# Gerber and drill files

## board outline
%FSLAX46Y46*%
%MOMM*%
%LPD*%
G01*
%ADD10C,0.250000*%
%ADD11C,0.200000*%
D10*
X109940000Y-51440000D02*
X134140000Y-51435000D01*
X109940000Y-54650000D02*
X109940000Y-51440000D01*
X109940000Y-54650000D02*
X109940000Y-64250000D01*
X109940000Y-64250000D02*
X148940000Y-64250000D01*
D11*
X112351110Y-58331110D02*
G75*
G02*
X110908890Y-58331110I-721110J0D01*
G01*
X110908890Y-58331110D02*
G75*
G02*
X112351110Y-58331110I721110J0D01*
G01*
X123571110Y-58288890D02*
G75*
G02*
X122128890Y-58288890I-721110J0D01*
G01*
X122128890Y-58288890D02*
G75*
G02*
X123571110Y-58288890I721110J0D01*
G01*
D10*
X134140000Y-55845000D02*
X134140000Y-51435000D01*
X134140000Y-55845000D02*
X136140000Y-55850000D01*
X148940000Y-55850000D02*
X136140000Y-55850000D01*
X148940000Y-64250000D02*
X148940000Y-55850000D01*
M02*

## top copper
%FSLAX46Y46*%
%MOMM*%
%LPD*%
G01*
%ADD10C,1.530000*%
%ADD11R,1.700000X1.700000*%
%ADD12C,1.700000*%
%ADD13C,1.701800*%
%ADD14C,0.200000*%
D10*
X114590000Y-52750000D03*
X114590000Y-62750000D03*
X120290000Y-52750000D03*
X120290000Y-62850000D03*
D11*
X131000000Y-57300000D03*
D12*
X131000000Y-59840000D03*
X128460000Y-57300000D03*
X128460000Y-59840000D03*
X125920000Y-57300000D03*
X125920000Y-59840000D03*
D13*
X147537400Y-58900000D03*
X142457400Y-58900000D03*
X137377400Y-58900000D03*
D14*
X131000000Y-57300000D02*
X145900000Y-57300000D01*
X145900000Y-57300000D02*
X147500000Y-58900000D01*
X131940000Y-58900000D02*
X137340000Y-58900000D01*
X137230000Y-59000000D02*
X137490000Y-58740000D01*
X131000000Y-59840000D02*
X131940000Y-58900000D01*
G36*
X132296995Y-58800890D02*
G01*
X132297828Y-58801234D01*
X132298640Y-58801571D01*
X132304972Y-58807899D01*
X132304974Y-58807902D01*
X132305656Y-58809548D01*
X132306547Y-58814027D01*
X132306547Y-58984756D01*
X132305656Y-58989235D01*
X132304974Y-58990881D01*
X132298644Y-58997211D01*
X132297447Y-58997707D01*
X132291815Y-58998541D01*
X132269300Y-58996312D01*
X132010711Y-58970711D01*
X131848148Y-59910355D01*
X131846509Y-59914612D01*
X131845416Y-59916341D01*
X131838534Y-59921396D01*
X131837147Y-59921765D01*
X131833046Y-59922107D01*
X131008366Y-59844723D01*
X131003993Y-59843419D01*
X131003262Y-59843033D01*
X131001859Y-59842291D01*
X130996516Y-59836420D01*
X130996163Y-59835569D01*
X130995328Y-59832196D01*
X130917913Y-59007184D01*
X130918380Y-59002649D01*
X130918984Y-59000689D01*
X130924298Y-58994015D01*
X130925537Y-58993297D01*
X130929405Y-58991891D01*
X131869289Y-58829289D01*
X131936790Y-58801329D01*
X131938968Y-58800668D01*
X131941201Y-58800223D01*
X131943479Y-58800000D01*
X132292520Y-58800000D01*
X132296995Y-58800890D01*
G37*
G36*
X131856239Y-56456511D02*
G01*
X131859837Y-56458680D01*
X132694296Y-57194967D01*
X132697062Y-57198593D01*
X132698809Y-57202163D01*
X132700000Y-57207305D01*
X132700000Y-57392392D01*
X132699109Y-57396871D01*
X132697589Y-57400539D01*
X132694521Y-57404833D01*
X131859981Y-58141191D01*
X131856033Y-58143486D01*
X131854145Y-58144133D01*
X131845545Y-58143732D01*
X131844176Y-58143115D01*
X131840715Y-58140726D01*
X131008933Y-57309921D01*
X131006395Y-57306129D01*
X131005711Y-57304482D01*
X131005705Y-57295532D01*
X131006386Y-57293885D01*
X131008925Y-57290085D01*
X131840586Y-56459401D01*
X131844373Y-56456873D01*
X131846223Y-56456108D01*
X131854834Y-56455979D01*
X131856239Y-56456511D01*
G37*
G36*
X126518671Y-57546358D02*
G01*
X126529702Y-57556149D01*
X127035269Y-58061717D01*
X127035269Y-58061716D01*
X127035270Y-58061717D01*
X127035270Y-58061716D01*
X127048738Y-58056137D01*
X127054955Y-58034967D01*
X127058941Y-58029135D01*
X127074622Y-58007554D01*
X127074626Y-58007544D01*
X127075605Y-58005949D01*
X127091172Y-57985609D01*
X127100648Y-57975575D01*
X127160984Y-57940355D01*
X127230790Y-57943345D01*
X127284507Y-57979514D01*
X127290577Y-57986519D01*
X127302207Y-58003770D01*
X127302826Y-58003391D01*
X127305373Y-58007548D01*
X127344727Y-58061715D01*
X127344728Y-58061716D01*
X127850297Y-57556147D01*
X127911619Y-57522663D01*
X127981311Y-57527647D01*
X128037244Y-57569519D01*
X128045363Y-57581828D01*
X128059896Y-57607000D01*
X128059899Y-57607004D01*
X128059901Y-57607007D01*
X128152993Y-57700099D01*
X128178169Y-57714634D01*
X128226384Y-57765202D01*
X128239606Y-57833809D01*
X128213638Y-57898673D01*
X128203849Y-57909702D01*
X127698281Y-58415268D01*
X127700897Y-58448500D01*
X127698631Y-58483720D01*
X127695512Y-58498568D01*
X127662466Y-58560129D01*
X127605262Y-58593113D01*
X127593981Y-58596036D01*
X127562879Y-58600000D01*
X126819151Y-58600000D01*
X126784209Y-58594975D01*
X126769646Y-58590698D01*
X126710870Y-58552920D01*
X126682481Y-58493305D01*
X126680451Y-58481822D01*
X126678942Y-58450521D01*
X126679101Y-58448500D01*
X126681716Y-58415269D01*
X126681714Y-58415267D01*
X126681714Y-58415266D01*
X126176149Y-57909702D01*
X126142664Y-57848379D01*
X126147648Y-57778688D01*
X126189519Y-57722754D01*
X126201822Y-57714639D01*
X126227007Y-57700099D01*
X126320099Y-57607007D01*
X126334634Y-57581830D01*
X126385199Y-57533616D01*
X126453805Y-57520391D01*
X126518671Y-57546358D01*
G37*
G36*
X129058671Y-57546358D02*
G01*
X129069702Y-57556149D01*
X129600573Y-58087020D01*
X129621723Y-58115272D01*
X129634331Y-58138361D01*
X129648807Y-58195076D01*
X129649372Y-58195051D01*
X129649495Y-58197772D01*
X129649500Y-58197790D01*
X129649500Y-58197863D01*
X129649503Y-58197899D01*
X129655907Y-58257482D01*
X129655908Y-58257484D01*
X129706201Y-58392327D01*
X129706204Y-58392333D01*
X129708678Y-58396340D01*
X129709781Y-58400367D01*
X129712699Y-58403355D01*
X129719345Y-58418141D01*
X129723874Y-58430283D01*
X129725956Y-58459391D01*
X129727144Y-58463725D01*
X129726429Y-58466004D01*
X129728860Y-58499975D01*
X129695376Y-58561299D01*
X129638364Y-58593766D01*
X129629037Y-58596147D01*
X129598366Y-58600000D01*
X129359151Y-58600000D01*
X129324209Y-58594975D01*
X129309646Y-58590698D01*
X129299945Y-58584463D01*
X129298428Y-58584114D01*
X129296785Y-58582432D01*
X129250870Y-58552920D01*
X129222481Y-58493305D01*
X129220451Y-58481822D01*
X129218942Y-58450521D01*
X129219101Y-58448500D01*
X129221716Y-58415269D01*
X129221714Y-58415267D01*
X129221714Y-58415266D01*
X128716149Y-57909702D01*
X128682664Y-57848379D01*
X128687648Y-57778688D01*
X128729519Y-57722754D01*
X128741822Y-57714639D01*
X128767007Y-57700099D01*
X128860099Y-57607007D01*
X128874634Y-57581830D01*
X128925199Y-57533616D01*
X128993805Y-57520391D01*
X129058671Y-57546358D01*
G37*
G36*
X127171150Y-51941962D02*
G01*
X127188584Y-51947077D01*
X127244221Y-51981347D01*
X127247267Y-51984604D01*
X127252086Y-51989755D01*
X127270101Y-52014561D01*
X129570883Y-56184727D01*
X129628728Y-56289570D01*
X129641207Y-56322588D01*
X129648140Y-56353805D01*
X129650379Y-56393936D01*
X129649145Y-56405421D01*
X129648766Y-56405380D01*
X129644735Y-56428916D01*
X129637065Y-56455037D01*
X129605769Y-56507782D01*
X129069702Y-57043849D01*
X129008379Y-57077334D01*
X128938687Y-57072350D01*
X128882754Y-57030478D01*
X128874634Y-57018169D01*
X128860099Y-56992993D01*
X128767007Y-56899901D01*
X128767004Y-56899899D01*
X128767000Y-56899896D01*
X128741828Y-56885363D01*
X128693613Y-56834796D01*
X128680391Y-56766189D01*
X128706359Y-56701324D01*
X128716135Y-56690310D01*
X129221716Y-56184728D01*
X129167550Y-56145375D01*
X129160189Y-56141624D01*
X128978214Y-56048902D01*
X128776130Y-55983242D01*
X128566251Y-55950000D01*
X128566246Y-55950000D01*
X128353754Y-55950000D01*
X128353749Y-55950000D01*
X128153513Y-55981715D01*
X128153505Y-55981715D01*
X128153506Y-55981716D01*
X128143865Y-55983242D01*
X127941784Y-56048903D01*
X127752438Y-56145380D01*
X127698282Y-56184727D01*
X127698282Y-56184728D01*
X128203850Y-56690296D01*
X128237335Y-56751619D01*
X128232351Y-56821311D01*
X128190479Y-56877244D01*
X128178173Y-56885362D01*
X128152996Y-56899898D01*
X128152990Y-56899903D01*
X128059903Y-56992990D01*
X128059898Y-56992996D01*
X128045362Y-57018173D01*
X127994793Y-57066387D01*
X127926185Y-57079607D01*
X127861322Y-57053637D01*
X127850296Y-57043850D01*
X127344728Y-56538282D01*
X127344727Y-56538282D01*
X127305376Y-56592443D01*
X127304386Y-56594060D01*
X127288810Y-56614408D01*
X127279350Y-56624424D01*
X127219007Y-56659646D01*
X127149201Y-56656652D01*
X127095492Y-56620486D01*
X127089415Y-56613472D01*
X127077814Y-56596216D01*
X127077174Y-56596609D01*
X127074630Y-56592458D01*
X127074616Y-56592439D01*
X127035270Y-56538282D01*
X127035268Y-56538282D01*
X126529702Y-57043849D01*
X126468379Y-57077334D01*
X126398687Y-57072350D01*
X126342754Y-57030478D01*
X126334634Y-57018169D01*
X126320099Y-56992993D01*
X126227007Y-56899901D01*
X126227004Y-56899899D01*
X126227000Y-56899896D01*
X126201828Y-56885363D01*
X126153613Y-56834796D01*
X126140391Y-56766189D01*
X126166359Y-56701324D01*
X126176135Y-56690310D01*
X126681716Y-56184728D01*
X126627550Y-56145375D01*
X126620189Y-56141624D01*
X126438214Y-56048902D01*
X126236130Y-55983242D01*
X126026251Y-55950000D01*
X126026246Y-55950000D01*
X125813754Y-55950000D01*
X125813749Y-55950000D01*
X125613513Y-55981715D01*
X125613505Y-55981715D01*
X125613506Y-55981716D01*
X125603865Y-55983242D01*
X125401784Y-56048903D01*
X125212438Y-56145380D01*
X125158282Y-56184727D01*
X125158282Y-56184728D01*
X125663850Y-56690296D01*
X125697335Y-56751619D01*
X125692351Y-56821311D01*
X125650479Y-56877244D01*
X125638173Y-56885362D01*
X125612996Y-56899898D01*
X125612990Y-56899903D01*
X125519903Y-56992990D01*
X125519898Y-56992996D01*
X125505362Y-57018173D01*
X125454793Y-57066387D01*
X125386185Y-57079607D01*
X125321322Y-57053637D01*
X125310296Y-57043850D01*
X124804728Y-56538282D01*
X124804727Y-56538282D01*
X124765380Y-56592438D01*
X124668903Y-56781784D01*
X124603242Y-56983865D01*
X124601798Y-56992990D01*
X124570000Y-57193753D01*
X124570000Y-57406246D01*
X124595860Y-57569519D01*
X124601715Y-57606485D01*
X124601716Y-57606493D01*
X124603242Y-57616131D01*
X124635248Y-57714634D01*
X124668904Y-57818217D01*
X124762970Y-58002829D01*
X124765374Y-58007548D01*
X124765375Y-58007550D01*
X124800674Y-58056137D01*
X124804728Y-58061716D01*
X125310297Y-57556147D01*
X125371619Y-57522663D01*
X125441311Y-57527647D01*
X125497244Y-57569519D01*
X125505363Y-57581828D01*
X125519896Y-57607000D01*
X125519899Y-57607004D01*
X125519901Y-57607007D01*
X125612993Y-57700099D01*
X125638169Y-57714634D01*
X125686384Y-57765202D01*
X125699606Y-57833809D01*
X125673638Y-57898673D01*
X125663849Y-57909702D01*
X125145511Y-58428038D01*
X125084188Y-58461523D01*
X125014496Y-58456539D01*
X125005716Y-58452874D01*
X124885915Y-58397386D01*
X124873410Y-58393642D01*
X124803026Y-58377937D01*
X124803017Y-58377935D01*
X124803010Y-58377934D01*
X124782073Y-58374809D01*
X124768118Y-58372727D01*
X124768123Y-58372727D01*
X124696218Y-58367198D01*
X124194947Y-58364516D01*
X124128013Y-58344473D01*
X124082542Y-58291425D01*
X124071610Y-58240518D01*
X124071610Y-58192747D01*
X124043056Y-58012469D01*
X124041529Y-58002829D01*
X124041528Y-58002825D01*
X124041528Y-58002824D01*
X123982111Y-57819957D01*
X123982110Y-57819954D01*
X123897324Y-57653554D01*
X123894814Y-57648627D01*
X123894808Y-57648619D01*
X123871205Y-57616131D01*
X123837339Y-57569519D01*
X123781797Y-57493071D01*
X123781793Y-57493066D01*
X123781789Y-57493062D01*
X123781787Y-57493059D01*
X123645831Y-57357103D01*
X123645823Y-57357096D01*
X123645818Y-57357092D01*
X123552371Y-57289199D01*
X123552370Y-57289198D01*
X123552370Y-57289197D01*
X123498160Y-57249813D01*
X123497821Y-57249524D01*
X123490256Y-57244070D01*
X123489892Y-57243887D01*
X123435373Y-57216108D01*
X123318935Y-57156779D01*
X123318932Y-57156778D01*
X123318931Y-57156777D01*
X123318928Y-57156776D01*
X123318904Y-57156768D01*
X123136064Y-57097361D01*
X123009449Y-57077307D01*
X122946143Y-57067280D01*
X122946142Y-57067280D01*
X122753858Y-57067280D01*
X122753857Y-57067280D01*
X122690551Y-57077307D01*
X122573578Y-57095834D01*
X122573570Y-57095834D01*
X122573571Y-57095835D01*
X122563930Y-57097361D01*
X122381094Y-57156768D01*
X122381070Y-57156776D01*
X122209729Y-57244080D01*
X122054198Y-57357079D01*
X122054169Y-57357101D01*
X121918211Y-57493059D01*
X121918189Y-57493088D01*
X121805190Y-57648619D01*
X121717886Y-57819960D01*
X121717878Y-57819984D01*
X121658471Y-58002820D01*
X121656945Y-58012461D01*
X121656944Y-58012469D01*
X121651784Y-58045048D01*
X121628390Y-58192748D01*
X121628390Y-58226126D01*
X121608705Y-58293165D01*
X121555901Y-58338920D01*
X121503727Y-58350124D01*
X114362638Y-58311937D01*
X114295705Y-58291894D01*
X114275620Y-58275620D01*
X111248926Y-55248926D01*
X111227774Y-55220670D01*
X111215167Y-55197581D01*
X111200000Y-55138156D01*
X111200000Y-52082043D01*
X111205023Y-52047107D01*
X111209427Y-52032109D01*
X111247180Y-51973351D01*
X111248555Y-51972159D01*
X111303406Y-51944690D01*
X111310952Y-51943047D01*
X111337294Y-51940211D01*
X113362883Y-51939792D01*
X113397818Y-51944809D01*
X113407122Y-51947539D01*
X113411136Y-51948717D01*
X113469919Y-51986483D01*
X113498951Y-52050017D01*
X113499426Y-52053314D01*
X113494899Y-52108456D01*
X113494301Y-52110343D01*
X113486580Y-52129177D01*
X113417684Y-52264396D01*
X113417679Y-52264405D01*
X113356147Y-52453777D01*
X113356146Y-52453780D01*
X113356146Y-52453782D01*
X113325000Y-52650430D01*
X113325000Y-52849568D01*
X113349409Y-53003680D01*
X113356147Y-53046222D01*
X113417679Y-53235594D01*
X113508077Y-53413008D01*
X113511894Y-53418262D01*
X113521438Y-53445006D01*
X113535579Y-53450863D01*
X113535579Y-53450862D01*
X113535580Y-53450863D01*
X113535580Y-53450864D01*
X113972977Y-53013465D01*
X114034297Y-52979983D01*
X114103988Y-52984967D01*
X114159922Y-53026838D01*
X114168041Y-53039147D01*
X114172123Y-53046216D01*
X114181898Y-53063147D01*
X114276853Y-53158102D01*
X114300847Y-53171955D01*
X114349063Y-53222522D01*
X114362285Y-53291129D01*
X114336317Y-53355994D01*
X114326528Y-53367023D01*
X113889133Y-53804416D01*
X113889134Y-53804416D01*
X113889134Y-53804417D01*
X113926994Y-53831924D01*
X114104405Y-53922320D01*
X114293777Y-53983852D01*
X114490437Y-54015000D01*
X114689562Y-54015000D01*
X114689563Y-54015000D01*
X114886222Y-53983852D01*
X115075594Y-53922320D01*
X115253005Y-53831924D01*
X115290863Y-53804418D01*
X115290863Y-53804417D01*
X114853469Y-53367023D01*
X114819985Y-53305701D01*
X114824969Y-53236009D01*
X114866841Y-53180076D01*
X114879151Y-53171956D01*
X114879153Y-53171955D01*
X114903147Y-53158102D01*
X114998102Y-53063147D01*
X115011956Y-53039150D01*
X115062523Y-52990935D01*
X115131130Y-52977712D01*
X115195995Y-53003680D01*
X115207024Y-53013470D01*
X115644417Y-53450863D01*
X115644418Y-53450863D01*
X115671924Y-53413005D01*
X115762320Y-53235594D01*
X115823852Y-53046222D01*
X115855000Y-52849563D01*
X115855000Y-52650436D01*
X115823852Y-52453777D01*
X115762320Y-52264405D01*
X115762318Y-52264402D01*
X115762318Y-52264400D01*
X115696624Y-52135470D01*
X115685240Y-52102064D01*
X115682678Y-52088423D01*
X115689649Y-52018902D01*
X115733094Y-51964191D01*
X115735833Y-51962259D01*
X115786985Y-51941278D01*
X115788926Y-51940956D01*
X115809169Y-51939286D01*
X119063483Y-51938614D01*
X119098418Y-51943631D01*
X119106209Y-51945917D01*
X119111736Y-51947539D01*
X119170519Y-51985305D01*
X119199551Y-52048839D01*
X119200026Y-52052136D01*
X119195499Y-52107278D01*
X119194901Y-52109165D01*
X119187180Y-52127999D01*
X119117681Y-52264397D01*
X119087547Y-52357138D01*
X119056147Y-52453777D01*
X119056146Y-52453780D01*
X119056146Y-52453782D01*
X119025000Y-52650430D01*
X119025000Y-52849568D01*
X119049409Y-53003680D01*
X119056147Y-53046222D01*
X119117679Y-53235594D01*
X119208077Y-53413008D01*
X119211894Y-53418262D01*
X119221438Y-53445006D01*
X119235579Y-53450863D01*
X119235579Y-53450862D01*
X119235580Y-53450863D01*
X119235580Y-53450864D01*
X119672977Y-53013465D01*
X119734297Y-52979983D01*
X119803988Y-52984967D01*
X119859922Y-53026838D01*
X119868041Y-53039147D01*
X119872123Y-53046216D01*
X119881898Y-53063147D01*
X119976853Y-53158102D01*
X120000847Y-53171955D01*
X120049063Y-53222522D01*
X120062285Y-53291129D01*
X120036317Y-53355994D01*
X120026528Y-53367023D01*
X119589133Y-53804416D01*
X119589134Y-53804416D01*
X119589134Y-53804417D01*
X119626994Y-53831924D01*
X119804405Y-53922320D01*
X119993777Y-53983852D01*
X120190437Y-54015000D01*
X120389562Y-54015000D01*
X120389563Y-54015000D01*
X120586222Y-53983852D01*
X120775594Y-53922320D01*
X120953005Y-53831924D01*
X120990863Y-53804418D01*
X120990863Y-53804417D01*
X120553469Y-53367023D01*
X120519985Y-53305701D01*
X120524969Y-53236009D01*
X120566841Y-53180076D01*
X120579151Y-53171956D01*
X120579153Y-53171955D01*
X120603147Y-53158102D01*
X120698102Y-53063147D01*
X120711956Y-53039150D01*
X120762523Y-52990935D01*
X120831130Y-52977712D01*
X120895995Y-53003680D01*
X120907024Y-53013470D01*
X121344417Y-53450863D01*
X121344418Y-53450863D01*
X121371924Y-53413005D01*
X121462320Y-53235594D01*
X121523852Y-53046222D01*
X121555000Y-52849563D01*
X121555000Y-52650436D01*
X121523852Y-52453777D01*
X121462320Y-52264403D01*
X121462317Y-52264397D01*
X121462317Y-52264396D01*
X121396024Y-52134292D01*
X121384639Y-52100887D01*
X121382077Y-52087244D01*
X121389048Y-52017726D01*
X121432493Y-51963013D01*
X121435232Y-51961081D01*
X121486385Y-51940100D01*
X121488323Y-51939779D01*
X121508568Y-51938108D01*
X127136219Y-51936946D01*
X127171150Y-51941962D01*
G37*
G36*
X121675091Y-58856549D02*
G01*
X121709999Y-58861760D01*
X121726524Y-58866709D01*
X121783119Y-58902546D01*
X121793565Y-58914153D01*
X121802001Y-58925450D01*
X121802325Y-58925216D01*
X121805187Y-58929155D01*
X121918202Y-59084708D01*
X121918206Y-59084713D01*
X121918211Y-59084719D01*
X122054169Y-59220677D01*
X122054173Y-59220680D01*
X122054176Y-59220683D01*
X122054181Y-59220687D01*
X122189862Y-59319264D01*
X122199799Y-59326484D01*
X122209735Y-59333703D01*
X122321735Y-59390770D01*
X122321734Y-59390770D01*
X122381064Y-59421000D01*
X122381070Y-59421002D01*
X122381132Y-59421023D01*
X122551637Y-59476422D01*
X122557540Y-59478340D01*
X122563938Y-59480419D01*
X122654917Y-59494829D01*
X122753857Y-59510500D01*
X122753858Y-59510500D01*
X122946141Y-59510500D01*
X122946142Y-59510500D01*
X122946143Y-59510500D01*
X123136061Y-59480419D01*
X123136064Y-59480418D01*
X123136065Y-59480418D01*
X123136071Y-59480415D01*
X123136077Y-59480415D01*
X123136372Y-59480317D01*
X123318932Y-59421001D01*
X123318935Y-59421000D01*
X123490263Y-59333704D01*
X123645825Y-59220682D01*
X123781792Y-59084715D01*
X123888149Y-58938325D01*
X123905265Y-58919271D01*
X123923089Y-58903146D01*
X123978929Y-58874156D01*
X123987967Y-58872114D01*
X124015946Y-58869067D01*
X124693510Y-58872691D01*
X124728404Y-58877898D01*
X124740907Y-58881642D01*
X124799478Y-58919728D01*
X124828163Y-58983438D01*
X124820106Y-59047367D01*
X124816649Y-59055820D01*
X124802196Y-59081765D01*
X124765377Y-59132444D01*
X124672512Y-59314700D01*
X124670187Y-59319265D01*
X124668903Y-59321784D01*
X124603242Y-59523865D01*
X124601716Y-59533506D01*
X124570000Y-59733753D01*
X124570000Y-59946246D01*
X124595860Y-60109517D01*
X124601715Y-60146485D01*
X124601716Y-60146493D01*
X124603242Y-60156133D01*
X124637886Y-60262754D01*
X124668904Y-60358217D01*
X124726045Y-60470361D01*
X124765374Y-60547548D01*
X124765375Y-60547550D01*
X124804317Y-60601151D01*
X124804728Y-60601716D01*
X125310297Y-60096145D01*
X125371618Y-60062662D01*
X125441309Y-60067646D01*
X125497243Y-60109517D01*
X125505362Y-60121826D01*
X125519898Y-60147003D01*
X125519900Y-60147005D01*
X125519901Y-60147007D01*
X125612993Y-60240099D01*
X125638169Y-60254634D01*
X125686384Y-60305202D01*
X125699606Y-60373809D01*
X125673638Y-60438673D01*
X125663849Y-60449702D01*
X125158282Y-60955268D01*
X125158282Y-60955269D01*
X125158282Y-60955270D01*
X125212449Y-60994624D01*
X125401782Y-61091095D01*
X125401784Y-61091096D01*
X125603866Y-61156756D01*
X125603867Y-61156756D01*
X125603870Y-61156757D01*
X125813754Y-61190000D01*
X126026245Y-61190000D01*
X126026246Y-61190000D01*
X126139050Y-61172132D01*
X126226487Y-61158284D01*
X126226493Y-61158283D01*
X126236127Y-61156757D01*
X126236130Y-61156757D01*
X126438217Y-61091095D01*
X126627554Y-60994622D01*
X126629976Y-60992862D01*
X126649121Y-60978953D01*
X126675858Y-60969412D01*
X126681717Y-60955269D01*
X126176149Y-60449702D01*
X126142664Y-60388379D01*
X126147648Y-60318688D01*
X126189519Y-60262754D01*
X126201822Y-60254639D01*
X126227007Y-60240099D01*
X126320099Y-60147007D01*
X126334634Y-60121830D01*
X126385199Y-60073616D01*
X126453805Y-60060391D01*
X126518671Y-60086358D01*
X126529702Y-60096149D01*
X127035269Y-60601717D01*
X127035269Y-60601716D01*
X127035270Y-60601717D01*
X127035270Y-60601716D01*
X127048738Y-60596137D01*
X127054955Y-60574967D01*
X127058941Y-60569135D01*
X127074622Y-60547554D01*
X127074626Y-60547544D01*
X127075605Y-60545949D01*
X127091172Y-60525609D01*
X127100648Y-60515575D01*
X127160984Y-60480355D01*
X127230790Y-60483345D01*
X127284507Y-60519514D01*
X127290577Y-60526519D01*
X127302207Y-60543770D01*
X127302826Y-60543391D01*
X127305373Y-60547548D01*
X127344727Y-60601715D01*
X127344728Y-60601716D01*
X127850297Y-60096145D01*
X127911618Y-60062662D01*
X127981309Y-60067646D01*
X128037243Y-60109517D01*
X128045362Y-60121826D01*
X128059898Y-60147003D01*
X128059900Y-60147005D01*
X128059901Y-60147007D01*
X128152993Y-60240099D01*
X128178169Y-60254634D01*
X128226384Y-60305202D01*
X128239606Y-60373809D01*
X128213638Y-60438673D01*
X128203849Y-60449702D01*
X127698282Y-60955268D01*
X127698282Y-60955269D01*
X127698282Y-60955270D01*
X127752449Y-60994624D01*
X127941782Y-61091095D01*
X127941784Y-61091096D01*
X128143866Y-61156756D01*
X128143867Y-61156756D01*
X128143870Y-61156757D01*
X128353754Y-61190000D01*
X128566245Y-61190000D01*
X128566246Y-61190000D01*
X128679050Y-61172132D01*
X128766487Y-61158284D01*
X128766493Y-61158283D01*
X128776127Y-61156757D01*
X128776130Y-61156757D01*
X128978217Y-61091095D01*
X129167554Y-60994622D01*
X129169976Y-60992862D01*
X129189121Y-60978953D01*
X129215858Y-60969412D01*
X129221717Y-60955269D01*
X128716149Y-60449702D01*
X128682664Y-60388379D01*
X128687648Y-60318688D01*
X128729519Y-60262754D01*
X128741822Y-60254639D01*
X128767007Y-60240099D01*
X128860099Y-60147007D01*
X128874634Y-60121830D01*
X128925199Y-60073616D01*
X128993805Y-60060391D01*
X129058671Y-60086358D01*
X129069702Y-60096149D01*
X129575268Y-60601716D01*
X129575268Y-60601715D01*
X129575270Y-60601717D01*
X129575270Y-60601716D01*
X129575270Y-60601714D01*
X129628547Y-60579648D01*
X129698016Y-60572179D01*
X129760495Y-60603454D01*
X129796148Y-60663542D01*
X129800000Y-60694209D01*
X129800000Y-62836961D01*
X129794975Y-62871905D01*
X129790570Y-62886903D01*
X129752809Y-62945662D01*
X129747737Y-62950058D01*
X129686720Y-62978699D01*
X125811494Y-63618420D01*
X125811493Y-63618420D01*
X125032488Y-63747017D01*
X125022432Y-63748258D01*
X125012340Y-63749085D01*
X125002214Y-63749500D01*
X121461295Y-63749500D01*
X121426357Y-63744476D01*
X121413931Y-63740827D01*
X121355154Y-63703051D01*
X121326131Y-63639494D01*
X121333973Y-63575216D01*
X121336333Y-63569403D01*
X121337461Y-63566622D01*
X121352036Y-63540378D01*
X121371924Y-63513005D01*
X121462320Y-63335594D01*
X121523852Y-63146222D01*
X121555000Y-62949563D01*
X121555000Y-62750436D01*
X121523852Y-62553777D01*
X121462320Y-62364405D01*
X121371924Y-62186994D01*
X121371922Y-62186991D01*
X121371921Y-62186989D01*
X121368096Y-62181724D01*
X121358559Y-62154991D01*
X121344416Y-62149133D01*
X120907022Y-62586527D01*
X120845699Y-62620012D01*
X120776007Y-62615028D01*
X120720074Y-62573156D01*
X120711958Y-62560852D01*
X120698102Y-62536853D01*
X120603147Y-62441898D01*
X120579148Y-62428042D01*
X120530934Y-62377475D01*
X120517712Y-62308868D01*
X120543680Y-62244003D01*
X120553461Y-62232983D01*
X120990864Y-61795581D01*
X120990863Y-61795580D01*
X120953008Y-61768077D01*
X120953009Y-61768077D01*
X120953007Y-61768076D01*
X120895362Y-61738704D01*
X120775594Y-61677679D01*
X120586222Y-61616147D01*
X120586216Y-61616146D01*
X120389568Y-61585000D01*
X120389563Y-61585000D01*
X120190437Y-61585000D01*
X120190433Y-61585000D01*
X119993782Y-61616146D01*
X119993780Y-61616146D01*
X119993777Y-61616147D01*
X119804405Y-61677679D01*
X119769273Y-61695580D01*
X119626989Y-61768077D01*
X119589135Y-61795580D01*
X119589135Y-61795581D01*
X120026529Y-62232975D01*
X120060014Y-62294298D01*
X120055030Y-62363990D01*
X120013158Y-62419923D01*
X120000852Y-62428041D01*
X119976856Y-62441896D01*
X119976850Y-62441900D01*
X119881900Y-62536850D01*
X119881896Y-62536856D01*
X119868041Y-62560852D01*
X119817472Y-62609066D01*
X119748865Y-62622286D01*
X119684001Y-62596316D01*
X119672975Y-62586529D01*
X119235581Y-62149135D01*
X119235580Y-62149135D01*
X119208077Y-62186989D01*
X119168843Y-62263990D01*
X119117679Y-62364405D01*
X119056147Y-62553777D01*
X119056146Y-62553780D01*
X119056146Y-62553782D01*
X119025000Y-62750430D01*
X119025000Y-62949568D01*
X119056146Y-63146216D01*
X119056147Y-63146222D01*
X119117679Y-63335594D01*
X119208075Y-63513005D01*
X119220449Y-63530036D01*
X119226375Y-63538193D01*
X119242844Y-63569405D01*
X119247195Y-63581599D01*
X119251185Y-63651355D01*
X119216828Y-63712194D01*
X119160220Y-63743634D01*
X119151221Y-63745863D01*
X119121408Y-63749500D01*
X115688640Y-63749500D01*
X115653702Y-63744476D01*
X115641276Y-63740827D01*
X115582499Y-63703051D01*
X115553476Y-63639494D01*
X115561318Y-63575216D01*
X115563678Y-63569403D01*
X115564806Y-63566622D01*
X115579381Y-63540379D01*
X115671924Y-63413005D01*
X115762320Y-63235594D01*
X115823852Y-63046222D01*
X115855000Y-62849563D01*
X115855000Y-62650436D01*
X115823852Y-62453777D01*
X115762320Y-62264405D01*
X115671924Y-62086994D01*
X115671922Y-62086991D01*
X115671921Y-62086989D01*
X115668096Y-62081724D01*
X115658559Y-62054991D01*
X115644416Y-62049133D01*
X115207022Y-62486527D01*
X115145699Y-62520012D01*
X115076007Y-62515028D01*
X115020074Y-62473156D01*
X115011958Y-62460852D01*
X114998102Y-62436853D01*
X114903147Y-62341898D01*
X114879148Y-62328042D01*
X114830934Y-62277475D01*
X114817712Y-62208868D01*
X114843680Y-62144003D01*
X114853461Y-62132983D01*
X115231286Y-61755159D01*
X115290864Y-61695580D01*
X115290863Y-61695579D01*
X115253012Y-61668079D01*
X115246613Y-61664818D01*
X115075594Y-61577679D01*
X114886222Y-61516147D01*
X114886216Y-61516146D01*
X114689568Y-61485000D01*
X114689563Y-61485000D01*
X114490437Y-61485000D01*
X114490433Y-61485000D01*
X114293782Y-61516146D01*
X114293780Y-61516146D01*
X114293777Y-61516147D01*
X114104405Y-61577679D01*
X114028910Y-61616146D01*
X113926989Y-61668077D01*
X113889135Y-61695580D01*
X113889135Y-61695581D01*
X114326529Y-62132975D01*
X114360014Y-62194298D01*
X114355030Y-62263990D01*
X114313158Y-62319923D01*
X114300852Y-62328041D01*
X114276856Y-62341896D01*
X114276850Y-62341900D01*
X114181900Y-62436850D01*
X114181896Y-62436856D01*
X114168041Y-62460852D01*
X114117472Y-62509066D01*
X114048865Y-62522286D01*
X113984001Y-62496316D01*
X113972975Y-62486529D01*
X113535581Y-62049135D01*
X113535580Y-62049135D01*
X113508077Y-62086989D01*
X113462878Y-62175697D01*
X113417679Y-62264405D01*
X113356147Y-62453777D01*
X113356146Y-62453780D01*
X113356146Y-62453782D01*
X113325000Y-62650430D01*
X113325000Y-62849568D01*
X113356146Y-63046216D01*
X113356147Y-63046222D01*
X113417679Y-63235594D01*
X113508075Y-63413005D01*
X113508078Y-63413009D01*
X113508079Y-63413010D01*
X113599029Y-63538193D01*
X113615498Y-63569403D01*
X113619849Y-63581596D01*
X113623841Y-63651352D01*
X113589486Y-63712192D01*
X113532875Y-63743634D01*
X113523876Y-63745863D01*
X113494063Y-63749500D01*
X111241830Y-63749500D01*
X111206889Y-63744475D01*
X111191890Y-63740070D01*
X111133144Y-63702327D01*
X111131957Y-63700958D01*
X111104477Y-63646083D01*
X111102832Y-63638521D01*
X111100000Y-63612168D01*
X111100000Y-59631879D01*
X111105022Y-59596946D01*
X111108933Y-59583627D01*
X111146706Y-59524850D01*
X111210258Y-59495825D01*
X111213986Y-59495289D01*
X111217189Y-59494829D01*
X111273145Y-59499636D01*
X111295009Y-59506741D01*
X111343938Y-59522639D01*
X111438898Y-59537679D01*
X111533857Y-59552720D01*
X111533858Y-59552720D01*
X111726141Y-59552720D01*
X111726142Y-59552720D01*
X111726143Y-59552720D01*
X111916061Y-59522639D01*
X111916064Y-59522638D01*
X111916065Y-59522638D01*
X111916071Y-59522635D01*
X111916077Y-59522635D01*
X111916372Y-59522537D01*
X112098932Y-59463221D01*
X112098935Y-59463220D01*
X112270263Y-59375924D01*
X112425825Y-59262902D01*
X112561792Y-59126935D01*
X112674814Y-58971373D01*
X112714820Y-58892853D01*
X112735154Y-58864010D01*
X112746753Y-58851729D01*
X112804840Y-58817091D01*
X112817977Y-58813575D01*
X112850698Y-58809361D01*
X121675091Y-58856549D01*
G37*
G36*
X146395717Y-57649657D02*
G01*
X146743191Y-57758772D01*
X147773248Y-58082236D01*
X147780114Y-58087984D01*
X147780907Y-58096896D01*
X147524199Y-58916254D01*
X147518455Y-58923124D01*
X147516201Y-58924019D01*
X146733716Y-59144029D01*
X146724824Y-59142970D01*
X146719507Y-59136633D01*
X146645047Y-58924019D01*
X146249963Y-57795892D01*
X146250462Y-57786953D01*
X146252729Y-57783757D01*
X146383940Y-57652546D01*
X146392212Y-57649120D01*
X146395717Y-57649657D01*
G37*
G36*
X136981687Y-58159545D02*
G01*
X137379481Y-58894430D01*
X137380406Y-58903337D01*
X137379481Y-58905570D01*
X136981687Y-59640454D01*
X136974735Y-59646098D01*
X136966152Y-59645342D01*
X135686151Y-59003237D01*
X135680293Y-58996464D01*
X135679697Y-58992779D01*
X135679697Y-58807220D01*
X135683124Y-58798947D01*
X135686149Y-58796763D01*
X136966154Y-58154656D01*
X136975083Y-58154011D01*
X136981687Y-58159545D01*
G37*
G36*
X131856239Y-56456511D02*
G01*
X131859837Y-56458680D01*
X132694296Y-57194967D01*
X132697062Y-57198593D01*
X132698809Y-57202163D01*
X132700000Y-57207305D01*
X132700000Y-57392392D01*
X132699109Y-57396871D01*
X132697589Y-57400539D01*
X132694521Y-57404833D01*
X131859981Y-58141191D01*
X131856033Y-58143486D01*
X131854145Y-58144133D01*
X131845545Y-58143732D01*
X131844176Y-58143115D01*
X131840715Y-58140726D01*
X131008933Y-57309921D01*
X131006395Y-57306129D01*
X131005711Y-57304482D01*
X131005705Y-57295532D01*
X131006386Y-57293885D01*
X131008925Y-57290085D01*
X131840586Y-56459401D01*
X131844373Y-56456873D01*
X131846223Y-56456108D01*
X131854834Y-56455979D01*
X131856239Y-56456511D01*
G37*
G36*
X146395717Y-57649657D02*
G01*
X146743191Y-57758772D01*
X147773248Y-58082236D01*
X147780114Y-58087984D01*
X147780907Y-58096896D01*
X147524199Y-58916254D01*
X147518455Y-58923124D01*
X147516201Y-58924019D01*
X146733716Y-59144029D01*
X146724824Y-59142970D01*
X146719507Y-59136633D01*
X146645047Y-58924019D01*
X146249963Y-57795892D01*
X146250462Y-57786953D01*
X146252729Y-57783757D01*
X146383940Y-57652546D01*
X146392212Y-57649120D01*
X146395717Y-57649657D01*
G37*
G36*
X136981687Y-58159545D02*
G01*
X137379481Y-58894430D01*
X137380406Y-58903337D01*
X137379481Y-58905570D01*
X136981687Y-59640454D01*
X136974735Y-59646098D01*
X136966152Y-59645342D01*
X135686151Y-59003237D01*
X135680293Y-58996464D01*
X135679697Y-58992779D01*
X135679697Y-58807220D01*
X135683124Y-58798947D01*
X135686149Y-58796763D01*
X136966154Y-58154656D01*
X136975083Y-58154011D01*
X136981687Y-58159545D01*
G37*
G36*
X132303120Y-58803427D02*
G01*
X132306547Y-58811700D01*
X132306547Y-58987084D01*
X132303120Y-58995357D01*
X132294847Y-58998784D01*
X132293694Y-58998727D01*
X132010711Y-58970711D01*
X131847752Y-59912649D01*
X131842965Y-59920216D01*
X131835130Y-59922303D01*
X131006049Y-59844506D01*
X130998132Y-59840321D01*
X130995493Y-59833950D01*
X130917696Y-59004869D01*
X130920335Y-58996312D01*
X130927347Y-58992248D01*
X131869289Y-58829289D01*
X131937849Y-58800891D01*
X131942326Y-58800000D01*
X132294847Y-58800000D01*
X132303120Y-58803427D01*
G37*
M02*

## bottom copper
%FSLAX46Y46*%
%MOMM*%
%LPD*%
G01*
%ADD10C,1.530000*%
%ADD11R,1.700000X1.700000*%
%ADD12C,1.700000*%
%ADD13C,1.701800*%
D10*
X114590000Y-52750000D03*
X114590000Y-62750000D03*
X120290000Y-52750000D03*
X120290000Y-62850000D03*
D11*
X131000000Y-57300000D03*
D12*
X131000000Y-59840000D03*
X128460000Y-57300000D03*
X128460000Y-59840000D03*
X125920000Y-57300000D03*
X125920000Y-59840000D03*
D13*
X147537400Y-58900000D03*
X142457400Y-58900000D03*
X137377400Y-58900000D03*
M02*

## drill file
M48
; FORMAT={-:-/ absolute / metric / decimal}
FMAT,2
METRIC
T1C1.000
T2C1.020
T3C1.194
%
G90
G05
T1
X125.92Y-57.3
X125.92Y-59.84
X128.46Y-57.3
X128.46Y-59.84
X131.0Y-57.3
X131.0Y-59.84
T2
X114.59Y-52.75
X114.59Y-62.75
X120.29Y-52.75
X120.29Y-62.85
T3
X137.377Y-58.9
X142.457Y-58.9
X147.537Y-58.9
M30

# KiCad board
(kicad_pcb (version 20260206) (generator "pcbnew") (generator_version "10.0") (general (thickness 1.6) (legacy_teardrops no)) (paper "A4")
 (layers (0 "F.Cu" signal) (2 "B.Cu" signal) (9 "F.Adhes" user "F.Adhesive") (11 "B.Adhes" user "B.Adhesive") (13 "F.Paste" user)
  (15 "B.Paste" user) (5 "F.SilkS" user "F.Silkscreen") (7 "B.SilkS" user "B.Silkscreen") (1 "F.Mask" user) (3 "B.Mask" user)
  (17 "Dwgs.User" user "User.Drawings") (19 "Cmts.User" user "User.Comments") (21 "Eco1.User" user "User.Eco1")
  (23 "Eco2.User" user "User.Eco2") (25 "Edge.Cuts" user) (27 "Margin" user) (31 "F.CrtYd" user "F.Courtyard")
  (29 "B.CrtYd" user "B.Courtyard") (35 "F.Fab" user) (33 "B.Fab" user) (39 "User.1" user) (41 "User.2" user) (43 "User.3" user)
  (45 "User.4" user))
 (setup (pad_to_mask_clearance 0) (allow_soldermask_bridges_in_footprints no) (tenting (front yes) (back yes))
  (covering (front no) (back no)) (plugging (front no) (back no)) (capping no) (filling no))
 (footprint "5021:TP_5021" (layer "F.Cu") (at 114.59 52.75 -90)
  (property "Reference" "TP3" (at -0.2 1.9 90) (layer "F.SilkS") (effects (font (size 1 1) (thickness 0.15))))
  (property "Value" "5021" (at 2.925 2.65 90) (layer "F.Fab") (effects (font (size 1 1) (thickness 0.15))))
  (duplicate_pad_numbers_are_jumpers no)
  (pad "TP" thru_hole circle (at 0 0 270) (size 1.53 1.53) (drill 1.02) (layers "*.Cu" "*.Mask") (remove_unused_layers no)
   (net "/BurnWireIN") (solder_mask_margin 0.102)
   (teardrops (best_length_ratio 0.5) (max_length 1) (best_width_ratio 1) (max_width 2) (curved_edges no) (filter_ratio 0.9) (enabled yes)
    (allow_two_segments yes) (prefer_zone_connections yes))))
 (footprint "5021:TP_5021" (layer "F.Cu") (at 114.59 62.75 -90)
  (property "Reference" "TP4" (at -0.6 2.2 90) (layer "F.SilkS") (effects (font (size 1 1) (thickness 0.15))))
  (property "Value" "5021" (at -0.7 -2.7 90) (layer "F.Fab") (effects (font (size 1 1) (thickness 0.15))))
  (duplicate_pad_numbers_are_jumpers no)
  (pad "TP" thru_hole circle (at 0 0 270) (size 1.53 1.53) (drill 1.02) (layers "*.Cu" "*.Mask") (remove_unused_layers no) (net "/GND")
   (solder_mask_margin 0.102)
   (teardrops (best_length_ratio 0.5) (max_length 1) (best_width_ratio 1) (max_width 2) (curved_edges no) (filter_ratio 0.9) (enabled yes)
    (allow_two_segments yes) (prefer_zone_connections yes))))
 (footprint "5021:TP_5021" (layer "F.Cu") (at 120.29 52.75 -90)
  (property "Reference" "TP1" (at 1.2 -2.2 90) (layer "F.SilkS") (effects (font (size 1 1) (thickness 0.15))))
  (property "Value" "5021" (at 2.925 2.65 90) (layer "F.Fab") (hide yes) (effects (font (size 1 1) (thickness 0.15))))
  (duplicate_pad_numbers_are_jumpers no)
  (pad "TP" thru_hole circle (at 0 0 270) (size 1.53 1.53) (drill 1.02) (layers "*.Cu" "*.Mask") (remove_unused_layers no)
   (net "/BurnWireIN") (solder_mask_margin 0.102)
   (teardrops (best_length_ratio 0.5) (max_length 1) (best_width_ratio 1) (max_width 2) (curved_edges no) (filter_ratio 0.9) (enabled yes)
    (allow_two_segments yes) (prefer_zone_connections yes))))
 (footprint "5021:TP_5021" (layer "F.Cu") (at 120.29 62.85 -90)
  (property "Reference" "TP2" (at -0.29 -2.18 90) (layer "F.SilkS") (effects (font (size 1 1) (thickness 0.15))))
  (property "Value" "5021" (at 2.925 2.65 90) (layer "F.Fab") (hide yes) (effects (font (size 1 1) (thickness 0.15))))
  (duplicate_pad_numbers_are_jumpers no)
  (pad "TP" thru_hole circle (at 0 0 270) (size 1.53 1.53) (drill 1.02) (layers "*.Cu" "*.Mask") (remove_unused_layers no) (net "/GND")
   (solder_mask_margin 0.102)
   (teardrops (best_length_ratio 0.5) (max_length 1) (best_width_ratio 1) (max_width 2) (curved_edges no) (filter_ratio 0.9) (enabled yes)
    (allow_two_segments yes) (prefer_zone_connections yes))))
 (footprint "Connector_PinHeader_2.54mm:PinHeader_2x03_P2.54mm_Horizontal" (layer "F.Cu") (at 131 57.3 -90)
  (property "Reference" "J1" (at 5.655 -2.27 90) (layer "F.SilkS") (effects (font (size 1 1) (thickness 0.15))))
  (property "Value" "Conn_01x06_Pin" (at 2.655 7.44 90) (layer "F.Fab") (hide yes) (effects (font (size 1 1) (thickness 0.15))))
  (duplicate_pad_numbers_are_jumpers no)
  (pad "1" thru_hole rect (at 0 0 270) (size 1.7 1.7) (drill 1) (layers "*.Cu" "*.Mask") (remove_unused_layers no)
   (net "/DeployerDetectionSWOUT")
   (teardrops (best_length_ratio 0.5) (max_length 1) (best_width_ratio 1) (max_width 2) (curved_edges no) (filter_ratio 0.9) (enabled yes)
    (allow_two_segments yes) (prefer_zone_connections yes)))
  (pad "2" thru_hole circle (at 2.54 0 270) (size 1.7 1.7) (drill 1) (layers "*.Cu" "*.Mask") (remove_unused_layers no)
   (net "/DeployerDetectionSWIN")
   (teardrops (best_length_ratio 0.5) (max_length 1) (best_width_ratio 1) (max_width 2) (curved_edges no) (filter_ratio 0.9) (enabled yes)
    (allow_two_segments yes) (prefer_zone_connections yes)))
  (pad "3" thru_hole circle (at 0 2.54 270) (size 1.7 1.7) (drill 1) (layers "*.Cu" "*.Mask") (remove_unused_layers no) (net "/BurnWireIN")
   (teardrops (best_length_ratio 0.5) (max_length 1) (best_width_ratio 1) (max_width 2) (curved_edges no) (filter_ratio 0.9) (enabled yes)
    (allow_two_segments yes) (prefer_zone_connections yes)))
  (pad "4" thru_hole circle (at 2.54 2.54 270) (size 1.7 1.7) (drill 1) (layers "*.Cu" "*.Mask") (remove_unused_layers no) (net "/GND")
   (teardrops (best_length_ratio 0.5) (max_length 1) (best_width_ratio 1) (max_width 2) (curved_edges no) (filter_ratio 0.9) (enabled yes)
    (allow_two_segments yes) (prefer_zone_connections yes)))
  (pad "5" thru_hole circle (at 0 5.08 270) (size 1.7 1.7) (drill 1) (layers "*.Cu" "*.Mask") (remove_unused_layers no) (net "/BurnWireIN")
   (teardrops (best_length_ratio 0.5) (max_length 1) (best_width_ratio 1) (max_width 2) (curved_edges no) (filter_ratio 0.9) (enabled yes)
    (allow_two_segments yes) (prefer_zone_connections yes)))
  (pad "6" thru_hole circle (at 2.54 5.08 270) (size 1.7 1.7) (drill 1) (layers "*.Cu" "*.Mask") (remove_unused_layers no) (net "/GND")
   (teardrops (best_length_ratio 0.5) (max_length 1) (best_width_ratio 1) (max_width 2) (curved_edges no) (filter_ratio 0.9) (enabled yes)
    (allow_two_segments yes) (prefer_zone_connections yes))))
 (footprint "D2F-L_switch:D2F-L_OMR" (layer "B.Cu") (at 147.5374 58.9 180)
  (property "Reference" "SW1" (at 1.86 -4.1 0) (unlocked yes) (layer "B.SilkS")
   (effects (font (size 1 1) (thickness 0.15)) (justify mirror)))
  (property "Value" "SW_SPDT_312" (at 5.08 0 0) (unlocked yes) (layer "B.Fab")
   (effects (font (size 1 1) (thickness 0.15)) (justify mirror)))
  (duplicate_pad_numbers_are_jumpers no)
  (pad "1" thru_hole circle (at 0 0 180) (size 1.7018 1.7018) (drill 1.1938) (layers "*.Cu" "*.Mask") (remove_unused_layers no)
   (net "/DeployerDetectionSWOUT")
   (teardrops (best_length_ratio 0.5) (max_length 1) (best_width_ratio 1) (max_width 2) (curved_edges no) (filter_ratio 0.9) (enabled yes)
    (allow_two_segments yes) (prefer_zone_connections yes)))
  (pad "2" thru_hole circle (at 5.08 0 180) (size 1.7018 1.7018) (drill 1.1938) (layers "*.Cu" "*.Mask") (remove_unused_layers no)
   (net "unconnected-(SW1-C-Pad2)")
   (teardrops (best_length_ratio 0.5) (max_length 1) (best_width_ratio 1) (max_width 2) (curved_edges no) (filter_ratio 0.9) (enabled yes)
    (allow_two_segments yes) (prefer_zone_connections yes)))
  (pad "3" thru_hole circle (at 10.16 0 180) (size 1.7018 1.7018) (drill 1.1938) (layers "*.Cu" "*.Mask") (remove_unused_layers no)
   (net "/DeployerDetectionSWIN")
   (teardrops (best_length_ratio 0.5) (max_length 1) (best_width_ratio 1) (max_width 2) (curved_edges no) (filter_ratio 0.9) (enabled yes)
    (allow_two_segments yes) (prefer_zone_connections yes))))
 (gr_line (start 109.94 51.44) (end 134.14 51.435) (stroke (width 0.25) (type solid)) (layer "Edge.Cuts"))
 (gr_line (start 109.94 54.65) (end 109.94 51.44) (stroke (width 0.25) (type solid)) (layer "Edge.Cuts"))
 (gr_line (start 109.94 54.65) (end 109.94 64.25) (stroke (width 0.25) (type default)) (layer "Edge.Cuts"))
 (gr_line (start 109.94 64.25) (end 148.94 64.25) (stroke (width 0.25) (type solid)) (layer "Edge.Cuts"))
 (gr_circle (center 111.63 58.33111) (end 112.23 58.73111) (stroke (width 0.2) (type solid)) (fill no) (layer "Edge.Cuts"))
 (gr_circle (center 122.85 58.28889) (end 123.45 58.68889) (stroke (width 0.2) (type solid)) (fill no) (layer "Edge.Cuts"))
 (gr_line (start 134.14 55.845) (end 134.14 51.435) (stroke (width 0.25) (type solid)) (layer "Edge.Cuts"))
 (gr_line (start 134.14 55.845) (end 136.14 55.85) (stroke (width 0.25) (type solid)) (layer "Edge.Cuts"))
 (gr_line (start 148.94 55.85) (end 136.14 55.85) (stroke (width 0.25) (type default)) (layer "Edge.Cuts"))
 (gr_line (start 148.94 64.25) (end 148.94 55.85) (stroke (width 0.25) (type default)) (layer "Edge.Cuts"))
 (segment (start 131 57.3) (end 145.9 57.3) (width 0.2) (layer "F.Cu") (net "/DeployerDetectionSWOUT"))
 (segment (start 145.9 57.3) (end 147.5 58.9) (width 0.2) (layer "F.Cu") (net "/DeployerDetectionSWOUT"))
 (segment (start 131.94 58.9) (end 137.34 58.9) (width 0.2) (layer "F.Cu") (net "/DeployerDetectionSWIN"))
 (segment (start 137.23 59) (end 137.49 58.74) (width 0.2) (layer "F.Cu") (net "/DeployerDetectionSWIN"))
 (segment (start 131 59.84) (end 131.94 58.9) (width 0.2) (layer "F.Cu") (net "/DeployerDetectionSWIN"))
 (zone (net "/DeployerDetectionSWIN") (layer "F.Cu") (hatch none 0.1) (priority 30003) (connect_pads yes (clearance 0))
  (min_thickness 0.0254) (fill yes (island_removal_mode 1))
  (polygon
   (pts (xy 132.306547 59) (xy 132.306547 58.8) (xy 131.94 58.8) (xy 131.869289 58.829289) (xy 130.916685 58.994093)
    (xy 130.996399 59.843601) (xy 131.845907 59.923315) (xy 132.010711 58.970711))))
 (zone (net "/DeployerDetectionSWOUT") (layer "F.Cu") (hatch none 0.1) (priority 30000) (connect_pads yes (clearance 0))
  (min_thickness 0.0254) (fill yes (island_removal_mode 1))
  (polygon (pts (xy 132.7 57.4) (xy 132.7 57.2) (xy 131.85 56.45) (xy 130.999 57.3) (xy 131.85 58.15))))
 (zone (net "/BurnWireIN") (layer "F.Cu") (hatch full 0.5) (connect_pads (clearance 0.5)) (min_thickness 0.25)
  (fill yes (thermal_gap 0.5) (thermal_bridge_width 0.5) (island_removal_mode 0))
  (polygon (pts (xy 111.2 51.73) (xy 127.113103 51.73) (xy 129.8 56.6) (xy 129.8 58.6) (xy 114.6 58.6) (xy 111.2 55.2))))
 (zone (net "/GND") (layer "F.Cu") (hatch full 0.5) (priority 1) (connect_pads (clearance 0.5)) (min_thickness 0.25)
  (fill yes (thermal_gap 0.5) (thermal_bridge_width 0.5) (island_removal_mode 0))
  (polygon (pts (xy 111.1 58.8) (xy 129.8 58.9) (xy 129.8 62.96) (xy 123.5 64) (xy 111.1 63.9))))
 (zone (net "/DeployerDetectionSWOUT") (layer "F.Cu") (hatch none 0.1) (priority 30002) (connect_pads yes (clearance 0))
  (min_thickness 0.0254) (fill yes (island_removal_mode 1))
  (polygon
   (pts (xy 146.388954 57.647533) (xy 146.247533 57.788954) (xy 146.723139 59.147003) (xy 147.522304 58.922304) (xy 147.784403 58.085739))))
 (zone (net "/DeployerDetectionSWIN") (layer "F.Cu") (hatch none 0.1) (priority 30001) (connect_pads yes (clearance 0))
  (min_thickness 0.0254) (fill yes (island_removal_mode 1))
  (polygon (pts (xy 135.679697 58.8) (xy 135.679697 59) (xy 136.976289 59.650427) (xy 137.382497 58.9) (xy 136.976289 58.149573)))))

